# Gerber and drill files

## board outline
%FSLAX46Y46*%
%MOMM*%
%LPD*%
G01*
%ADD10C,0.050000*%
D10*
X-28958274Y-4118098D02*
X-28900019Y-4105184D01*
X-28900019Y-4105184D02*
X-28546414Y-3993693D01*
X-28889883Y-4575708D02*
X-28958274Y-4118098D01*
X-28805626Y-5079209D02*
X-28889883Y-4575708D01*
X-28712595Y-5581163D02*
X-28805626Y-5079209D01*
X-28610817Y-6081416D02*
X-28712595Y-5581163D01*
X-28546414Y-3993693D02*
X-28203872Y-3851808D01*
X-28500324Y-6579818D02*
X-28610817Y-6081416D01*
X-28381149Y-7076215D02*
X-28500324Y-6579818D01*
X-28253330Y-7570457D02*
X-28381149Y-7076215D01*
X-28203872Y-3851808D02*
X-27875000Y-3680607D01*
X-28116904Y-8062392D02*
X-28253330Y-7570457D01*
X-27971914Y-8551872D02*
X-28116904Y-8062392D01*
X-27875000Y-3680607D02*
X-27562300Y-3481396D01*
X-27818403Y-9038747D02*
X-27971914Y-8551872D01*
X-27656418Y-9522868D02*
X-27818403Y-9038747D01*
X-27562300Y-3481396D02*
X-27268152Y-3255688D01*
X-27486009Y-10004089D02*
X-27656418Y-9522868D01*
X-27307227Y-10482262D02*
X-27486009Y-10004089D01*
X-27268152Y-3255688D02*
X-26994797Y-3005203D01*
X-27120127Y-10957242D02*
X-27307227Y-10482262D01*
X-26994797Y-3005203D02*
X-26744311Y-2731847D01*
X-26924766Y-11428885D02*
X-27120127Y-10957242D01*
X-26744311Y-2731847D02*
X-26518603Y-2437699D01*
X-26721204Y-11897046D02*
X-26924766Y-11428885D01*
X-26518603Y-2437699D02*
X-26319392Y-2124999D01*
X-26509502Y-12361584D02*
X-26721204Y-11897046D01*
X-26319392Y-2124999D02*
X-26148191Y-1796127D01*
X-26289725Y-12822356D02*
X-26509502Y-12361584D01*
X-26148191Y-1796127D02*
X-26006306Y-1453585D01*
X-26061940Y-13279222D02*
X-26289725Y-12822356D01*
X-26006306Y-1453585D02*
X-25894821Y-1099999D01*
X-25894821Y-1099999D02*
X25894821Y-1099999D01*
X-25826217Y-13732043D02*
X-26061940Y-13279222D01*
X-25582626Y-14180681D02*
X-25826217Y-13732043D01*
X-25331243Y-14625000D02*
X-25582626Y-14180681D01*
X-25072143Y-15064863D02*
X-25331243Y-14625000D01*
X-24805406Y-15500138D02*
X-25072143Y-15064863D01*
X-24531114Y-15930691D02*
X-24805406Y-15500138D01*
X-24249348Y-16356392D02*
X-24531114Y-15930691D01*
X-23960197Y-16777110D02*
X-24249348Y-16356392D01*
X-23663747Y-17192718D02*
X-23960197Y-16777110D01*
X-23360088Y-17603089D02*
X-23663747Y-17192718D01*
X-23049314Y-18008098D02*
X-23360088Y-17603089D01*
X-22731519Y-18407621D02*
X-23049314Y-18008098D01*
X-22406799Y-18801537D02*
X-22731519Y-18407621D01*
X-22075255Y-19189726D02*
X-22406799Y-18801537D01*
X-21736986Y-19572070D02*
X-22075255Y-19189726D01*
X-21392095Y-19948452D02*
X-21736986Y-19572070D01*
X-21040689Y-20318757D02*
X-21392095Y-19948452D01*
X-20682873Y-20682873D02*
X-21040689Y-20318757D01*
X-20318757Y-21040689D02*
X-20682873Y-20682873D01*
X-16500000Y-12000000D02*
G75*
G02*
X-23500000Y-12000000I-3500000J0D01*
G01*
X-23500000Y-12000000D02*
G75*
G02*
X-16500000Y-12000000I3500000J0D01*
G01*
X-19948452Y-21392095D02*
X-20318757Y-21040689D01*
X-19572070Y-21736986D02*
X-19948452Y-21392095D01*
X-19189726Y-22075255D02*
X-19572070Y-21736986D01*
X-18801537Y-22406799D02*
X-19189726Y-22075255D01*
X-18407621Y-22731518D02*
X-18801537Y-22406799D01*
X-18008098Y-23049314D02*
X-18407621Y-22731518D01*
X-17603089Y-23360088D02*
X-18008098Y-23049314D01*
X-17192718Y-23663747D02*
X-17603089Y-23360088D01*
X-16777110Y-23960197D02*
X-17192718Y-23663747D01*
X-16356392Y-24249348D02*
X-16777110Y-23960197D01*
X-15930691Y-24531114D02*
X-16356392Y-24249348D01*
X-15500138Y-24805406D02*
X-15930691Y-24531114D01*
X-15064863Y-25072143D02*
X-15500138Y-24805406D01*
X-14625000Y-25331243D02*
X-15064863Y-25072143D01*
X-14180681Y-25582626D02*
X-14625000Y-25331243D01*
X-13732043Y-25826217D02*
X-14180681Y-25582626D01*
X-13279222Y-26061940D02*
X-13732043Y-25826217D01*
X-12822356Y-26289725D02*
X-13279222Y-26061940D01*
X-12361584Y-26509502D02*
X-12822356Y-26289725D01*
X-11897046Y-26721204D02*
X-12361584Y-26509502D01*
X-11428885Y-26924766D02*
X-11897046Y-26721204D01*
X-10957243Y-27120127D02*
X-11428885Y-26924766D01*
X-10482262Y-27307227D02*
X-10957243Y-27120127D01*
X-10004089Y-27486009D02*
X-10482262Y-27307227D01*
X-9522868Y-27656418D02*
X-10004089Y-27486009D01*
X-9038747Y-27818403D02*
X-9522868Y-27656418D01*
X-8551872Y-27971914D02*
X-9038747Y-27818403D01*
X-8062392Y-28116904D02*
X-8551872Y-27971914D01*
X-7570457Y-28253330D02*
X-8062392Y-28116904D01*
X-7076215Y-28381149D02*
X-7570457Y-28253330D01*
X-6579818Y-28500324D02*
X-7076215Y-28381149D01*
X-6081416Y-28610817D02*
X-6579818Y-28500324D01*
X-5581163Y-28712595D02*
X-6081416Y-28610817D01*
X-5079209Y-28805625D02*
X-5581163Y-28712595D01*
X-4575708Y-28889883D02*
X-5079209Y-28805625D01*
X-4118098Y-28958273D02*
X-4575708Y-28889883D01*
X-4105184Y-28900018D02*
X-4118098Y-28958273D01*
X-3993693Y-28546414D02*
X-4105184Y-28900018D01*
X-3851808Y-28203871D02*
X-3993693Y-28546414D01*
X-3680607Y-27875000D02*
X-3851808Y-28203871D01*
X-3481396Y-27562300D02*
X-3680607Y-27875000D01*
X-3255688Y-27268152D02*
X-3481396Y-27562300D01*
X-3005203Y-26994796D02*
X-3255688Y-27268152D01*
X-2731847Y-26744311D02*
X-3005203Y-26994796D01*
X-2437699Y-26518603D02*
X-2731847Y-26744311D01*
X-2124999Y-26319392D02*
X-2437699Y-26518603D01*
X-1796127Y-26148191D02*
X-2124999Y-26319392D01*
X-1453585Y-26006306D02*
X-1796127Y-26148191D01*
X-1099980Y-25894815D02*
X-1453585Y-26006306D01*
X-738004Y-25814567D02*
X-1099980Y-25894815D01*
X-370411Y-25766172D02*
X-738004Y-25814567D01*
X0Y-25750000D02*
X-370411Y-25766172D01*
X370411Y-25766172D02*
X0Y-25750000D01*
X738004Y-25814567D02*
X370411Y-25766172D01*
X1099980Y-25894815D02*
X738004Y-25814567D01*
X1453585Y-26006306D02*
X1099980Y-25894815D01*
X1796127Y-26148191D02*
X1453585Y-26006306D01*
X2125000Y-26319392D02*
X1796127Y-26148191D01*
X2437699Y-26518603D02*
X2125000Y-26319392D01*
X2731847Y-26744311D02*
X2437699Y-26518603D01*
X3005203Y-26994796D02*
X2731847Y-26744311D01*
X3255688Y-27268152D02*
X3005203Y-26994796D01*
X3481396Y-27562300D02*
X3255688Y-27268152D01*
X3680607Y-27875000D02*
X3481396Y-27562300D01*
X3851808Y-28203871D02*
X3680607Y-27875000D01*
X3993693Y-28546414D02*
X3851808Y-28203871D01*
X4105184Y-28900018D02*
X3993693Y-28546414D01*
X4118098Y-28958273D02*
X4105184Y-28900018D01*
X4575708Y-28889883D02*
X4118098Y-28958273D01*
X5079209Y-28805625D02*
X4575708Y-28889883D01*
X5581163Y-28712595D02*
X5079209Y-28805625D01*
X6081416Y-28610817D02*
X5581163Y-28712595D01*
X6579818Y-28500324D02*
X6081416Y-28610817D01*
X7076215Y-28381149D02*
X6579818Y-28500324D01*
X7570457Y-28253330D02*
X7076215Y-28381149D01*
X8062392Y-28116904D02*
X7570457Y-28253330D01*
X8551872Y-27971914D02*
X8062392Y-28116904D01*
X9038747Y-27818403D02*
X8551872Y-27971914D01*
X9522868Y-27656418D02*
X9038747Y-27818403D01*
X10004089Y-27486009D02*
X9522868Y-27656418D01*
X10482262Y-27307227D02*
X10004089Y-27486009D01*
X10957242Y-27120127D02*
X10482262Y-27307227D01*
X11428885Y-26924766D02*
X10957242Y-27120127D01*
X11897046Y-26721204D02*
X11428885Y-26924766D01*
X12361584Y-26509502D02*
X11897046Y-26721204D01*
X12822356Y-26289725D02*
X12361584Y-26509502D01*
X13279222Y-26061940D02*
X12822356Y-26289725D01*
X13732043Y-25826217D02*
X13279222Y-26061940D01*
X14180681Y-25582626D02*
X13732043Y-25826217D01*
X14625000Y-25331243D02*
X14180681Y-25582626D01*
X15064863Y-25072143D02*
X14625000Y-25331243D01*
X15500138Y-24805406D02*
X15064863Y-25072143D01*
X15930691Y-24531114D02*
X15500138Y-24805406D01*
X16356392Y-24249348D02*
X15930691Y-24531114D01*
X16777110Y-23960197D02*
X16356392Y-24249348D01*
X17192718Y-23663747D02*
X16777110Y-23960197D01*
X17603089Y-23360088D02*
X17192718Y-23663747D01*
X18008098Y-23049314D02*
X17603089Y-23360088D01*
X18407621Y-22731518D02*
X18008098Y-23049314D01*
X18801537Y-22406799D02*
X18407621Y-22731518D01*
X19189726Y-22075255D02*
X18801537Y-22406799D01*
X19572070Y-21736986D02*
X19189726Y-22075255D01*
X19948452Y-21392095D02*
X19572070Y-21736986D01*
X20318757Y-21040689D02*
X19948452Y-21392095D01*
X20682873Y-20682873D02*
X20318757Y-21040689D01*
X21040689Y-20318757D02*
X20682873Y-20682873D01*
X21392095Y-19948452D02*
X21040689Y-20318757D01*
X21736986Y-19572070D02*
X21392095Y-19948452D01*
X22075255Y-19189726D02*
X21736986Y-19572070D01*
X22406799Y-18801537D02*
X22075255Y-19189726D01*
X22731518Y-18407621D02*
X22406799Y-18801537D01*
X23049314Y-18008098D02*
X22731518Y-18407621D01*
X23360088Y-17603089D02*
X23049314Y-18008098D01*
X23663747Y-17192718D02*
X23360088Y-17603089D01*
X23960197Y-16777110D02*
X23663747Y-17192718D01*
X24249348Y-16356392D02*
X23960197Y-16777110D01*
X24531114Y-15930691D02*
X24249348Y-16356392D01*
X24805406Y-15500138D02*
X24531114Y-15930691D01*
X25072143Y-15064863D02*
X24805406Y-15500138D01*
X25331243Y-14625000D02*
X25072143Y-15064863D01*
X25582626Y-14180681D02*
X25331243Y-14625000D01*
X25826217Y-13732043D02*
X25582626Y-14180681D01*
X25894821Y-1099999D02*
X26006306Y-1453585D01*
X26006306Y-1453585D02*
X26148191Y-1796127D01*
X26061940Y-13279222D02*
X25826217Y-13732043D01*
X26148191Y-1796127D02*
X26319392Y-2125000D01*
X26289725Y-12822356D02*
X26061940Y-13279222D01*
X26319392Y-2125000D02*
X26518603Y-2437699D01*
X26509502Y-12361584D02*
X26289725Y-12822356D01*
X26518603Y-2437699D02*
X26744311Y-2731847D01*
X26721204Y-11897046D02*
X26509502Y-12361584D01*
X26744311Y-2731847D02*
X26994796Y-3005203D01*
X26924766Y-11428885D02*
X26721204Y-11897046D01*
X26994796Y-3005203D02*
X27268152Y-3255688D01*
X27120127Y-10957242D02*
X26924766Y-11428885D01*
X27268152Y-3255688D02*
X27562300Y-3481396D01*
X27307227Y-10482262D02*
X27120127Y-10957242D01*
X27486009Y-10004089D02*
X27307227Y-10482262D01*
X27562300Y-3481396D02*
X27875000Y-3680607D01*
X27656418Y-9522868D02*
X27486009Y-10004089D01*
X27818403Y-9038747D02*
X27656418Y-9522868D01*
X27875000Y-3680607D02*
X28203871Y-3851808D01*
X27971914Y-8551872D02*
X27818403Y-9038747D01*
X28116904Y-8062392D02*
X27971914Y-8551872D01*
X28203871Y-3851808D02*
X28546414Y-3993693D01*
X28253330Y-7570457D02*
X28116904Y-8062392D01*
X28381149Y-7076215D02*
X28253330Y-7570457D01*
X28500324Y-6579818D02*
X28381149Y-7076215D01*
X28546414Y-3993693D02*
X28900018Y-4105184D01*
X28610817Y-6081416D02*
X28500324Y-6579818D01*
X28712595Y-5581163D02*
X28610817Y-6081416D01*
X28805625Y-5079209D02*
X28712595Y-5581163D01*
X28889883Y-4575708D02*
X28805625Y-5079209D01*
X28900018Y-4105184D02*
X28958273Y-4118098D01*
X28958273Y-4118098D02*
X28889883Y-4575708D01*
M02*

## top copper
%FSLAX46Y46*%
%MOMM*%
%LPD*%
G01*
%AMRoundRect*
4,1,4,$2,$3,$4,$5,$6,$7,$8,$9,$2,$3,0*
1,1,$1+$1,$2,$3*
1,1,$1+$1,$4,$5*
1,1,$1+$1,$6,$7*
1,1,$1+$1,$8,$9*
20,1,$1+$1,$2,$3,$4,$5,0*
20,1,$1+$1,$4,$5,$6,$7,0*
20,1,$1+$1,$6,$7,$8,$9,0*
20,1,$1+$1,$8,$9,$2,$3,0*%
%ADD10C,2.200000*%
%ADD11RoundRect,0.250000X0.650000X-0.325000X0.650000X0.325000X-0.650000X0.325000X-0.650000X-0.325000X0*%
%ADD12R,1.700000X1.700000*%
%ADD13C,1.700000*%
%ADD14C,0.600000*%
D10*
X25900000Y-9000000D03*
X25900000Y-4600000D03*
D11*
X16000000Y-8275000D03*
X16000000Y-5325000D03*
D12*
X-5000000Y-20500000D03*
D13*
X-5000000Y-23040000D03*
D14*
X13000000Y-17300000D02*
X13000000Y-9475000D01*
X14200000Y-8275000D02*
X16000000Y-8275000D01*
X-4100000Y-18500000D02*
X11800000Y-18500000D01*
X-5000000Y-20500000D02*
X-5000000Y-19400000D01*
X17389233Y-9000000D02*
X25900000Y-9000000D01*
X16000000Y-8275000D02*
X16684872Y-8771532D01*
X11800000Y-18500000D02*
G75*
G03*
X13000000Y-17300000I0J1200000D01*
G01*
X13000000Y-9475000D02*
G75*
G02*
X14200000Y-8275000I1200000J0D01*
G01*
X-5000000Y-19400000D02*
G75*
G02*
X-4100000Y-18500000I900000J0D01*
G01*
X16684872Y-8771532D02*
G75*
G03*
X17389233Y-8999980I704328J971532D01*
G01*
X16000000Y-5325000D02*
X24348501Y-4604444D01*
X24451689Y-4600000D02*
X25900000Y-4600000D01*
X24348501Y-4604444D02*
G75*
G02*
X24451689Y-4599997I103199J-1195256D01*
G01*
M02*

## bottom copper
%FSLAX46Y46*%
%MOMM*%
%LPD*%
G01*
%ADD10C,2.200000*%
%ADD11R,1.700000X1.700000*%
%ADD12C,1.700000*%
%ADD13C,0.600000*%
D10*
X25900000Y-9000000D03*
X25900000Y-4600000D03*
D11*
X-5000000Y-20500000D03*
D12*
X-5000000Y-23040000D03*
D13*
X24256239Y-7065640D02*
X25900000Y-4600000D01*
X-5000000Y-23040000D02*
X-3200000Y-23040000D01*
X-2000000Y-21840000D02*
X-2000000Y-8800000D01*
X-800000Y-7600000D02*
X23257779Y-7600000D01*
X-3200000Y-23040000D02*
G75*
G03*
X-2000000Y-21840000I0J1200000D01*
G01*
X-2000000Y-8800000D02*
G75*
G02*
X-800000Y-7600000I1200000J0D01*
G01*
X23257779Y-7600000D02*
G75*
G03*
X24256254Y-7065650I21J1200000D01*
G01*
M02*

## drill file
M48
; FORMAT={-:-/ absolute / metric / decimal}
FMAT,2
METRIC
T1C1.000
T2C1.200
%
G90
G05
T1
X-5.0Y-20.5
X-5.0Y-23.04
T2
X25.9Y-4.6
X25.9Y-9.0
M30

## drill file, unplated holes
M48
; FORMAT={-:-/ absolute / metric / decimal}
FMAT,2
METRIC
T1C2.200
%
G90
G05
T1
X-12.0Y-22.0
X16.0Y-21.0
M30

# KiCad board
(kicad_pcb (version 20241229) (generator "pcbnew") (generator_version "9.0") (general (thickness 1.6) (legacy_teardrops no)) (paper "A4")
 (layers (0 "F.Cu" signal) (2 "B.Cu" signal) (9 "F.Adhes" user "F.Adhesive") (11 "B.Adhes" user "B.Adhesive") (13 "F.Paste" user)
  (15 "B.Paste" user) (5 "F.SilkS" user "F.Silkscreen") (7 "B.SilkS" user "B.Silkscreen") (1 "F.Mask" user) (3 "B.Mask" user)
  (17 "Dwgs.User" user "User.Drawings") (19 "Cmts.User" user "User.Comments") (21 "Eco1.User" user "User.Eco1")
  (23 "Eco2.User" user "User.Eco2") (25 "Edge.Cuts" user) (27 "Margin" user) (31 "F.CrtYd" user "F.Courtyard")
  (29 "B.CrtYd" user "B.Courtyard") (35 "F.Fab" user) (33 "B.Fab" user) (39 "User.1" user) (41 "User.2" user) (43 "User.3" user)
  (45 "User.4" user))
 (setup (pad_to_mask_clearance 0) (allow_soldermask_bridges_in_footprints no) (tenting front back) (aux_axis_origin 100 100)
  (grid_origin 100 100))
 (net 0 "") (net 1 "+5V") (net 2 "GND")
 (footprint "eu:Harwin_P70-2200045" (layer "F.Cu") (at 125.9 109)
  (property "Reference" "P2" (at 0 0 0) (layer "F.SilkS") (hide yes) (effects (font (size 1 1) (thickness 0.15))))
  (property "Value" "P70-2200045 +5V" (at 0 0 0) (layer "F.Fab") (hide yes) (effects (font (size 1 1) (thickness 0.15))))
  (pad "1" thru_hole circle (at 0 0) (size 2.2 2.2) (drill 1.2) (layers "*.Cu" "*.Mask" "F.Paste") (remove_unused_layers no) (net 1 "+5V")))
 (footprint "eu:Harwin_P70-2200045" (layer "F.Cu") (at 125.9 104.6)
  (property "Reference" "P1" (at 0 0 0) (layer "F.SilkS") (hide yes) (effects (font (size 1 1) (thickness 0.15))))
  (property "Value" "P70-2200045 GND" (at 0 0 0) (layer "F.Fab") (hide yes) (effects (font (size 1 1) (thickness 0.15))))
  (pad "1" thru_hole circle (at 0 0) (size 2.2 2.2) (drill 1.2) (layers "*.Cu" "*.Mask" "F.Paste") (remove_unused_layers no) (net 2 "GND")))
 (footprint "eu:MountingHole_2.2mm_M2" (layer "F.Cu") (at 88 122)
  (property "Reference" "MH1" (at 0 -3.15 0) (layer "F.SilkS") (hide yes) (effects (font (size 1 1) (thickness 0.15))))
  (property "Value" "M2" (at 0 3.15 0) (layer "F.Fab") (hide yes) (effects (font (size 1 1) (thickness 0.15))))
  (pad "" np_thru_hole circle (at 0 0) (size 2.2 2.2) (drill 2.2) (layers "*.Cu" "*.Mask")))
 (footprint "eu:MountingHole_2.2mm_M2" (layer "F.Cu") (at 116 121)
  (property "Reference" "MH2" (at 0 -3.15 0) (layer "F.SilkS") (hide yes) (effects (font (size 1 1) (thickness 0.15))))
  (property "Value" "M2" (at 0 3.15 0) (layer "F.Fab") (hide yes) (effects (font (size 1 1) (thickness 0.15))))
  (pad "" np_thru_hole circle (at 0 0) (size 2.2 2.2) (drill 2.2) (layers "*.Cu" "*.Mask")))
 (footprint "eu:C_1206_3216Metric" (layer "F.Cu") (at 116 106.8 90)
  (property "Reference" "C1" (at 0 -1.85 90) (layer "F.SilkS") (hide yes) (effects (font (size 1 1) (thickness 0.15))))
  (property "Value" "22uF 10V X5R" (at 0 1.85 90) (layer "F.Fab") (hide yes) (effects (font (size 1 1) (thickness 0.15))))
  (pad "1" smd roundrect (at -1.475 0 90) (size 1.15 1.8) (layers "F.Cu" "F.Mask" "F.Paste") (roundrect_rratio 0.217391) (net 1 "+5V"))
  (pad "2" smd roundrect (at 1.475 0 90) (size 1.15 1.8) (layers "F.Cu" "F.Mask" "F.Paste") (roundrect_rratio 0.217391) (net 2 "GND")))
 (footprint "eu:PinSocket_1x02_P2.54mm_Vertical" (layer "B.Cu") (at 95 120.5 180)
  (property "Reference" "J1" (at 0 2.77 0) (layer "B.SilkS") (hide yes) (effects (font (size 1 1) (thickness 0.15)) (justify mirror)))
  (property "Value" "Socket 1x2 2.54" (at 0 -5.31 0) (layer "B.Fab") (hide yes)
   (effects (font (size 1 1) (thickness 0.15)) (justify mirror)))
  (pad "1" thru_hole rect (at 0 0 180) (size 1.7 1.7) (drill 1) (layers "*.Cu" "*.Mask") (remove_unused_layers no) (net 1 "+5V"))
  (pad "2" thru_hole circle (at 0 -2.54 180) (size 1.7 1.7) (drill 1) (layers "*.Cu" "*.Mask") (remove_unused_layers no) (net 2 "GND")))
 (gr_line (start 71.041726 104.118098) (end 71.099981 104.105184) (stroke (width 0.05) (type default)) (layer "Edge.Cuts"))
 (gr_line (start 71.099981 104.105184) (end 71.453586 103.993693) (stroke (width 0.05) (type default)) (layer "Edge.Cuts"))
 (gr_line (start 71.110117 104.575708) (end 71.041726 104.118098) (stroke (width 0.05) (type default)) (layer "Edge.Cuts"))
 (gr_line (start 71.194374 105.079209) (end 71.110117 104.575708) (stroke (width 0.05) (type default)) (layer "Edge.Cuts"))
 (gr_line (start 71.287405 105.581163) (end 71.194374 105.079209) (stroke (width 0.05) (type default)) (layer "Edge.Cuts"))
 (gr_line (start 71.389183 106.081416) (end 71.287405 105.581163) (stroke (width 0.05) (type default)) (layer "Edge.Cuts"))
 (gr_line (start 71.453586 103.993693) (end 71.796128 103.851808) (stroke (width 0.05) (type default)) (layer "Edge.Cuts"))
 (gr_line (start 71.499676 106.579818) (end 71.389183 106.081416) (stroke (width 0.05) (type default)) (layer "Edge.Cuts"))
 (gr_line (start 71.618851 107.076215) (end 71.499676 106.579818) (stroke (width 0.05) (type default)) (layer "Edge.Cuts"))
 (gr_line (start 71.74667 107.570457) (end 71.618851 107.076215) (stroke (width 0.05) (type default)) (layer "Edge.Cuts"))
 (gr_line (start 71.796128 103.851808) (end 72.125 103.680607) (stroke (width 0.05) (type default)) (layer "Edge.Cuts"))
 (gr_line (start 71.883096 108.062392) (end 71.74667 107.570457) (stroke (width 0.05) (type default)) (layer "Edge.Cuts"))
 (gr_line (start 72.028086 108.551872) (end 71.883096 108.062392) (stroke (width 0.05) (type default)) (layer "Edge.Cuts"))
 (gr_line (start 72.125 103.680607) (end 72.4377 103.481396) (stroke (width 0.05) (type default)) (layer "Edge.Cuts"))
 (gr_line (start 72.181597 109.038747) (end 72.028086 108.551872) (stroke (width 0.05) (type default)) (layer "Edge.Cuts"))
 (gr_line (start 72.343582 109.522868) (end 72.181597 109.038747) (stroke (width 0.05) (type default)) (layer "Edge.Cuts"))
 (gr_line (start 72.4377 103.481396) (end 72.731848 103.255688) (stroke (width 0.05) (type default)) (layer "Edge.Cuts"))
 (gr_line (start 72.513991 110.004089) (end 72.343582 109.522868) (stroke (width 0.05) (type default)) (layer "Edge.Cuts"))
 (gr_line (start 72.692773 110.482262) (end 72.513991 110.004089) (stroke (width 0.05) (type default)) (layer "Edge.Cuts"))
 (gr_line (start 72.731848 103.255688) (end 73.005203 103.005203) (stroke (width 0.05) (type default)) (layer "Edge.Cuts"))
 (gr_line (start 72.879873 110.957242) (end 72.692773 110.482262) (stroke (width 0.05) (type default)) (layer "Edge.Cuts"))
 (gr_line (start 73.005203 103.005203) (end 73.255689 102.731847) (stroke (width 0.05) (type default)) (layer "Edge.Cuts"))
 (gr_line (start 73.075234 111.428885) (end 72.879873 110.957242) (stroke (width 0.05) (type default)) (layer "Edge.Cuts"))
 (gr_line (start 73.255689 102.731847) (end 73.481397 102.437699) (stroke (width 0.05) (type default)) (layer "Edge.Cuts"))
 (gr_line (start 73.278796 111.897046) (end 73.075234 111.428885) (stroke (width 0.05) (type default)) (layer "Edge.Cuts"))
 (gr_line (start 73.481397 102.437699) (end 73.680608 102.124999) (stroke (width 0.05) (type default)) (layer "Edge.Cuts"))
 (gr_line (start 73.490498 112.361584) (end 73.278796 111.897046) (stroke (width 0.05) (type default)) (layer "Edge.Cuts"))
 (gr_line (start 73.680608 102.124999) (end 73.851809 101.796127) (stroke (width 0.05) (type default)) (layer "Edge.Cuts"))
 (gr_line (start 73.710275 112.822356) (end 73.490498 112.361584) (stroke (width 0.05) (type default)) (layer "Edge.Cuts"))
 (gr_line (start 73.851809 101.796127) (end 73.993694 101.453585) (stroke (width 0.05) (type default)) (layer "Edge.Cuts"))
 (gr_line (start 73.93806 113.279222) (end 73.710275 112.822356) (stroke (width 0.05) (type default)) (layer "Edge.Cuts"))
 (gr_line (start 73.993694 101.453585) (end 74.105179 101.099999) (stroke (width 0.05) (type default)) (layer "Edge.Cuts"))
 (gr_line (start 74.105179 101.099999) (end 125.894821 101.099999) (stroke (width 0.05) (type default)) (layer "Edge.Cuts"))
 (gr_line (start 74.173783 113.732043) (end 73.93806 113.279222) (stroke (width 0.05) (type default)) (layer "Edge.Cuts"))
 (gr_line (start 74.417374 114.180681) (end 74.173783 113.732043) (stroke (width 0.05) (type default)) (layer "Edge.Cuts"))
 (gr_line (start 74.668757 114.625) (end 74.417374 114.180681) (stroke (width 0.05) (type default)) (layer "Edge.Cuts"))
 (gr_line (start 74.927857 115.064863) (end 74.668757 114.625) (stroke (width 0.05) (type default)) (layer "Edge.Cuts"))
 (gr_line (start 75.194594 115.500138) (end 74.927857 115.064863) (stroke (width 0.05) (type default)) (layer "Edge.Cuts"))
 (gr_line (start 75.468886 115.930691) (end 75.194594 115.500138) (stroke (width 0.05) (type default)) (layer "Edge.Cuts"))
 (gr_line (start 75.750652 116.356392) (end 75.468886 115.930691) (stroke (width 0.05) (type default)) (layer "Edge.Cuts"))
 (gr_line (start 76.039803 116.77711) (end 75.750652 116.356392) (stroke (width 0.05) (type default)) (layer "Edge.Cuts"))
 (gr_line (start 76.336253 117.192718) (end 76.039803 116.77711) (stroke (width 0.05) (type default)) (layer "Edge.Cuts"))
 (gr_line (start 76.639912 117.603089) (end 76.336253 117.192718) (stroke (width 0.05) (type default)) (layer "Edge.Cuts"))
 (gr_line (start 76.950686 118.008098) (end 76.639912 117.603089) (stroke (width 0.05) (type default)) (layer "Edge.Cuts"))
 (gr_line (start 77.268481 118.407621) (end 76.950686 118.008098) (stroke (width 0.05) (type default)) (layer "Edge.Cuts"))
 (gr_line (start 77.593201 118.801537) (end 77.268481 118.407621) (stroke (width 0.05) (type default)) (layer "Edge.Cuts"))
 (gr_line (start 77.924745 119.189726) (end 77.593201 118.801537) (stroke (width 0.05) (type default)) (layer "Edge.Cuts"))
 (gr_line (start 78.263014 119.57207) (end 77.924745 119.189726) (stroke (width 0.05) (type default)) (layer "Edge.Cuts"))
 (gr_line (start 78.607905 119.948452) (end 78.263014 119.57207) (stroke (width 0.05) (type default)) (layer "Edge.Cuts"))
 (gr_line (start 78.959311 120.318757) (end 78.607905 119.948452) (stroke (width 0.05) (type default)) (layer "Edge.Cuts"))
 (gr_line (start 79.317127 120.682873) (end 78.959311 120.318757) (stroke (width 0.05) (type default)) (layer "Edge.Cuts"))
 (gr_line (start 79.681243 121.040689) (end 79.317127 120.682873) (stroke (width 0.05) (type default)) (layer "Edge.Cuts"))
 (gr_circle (center 80 112) (end 83.5 112) (stroke (width 0.05) (type default)) (fill no) (layer "Edge.Cuts"))
 (gr_line (start 80.051548 121.392095) (end 79.681243 121.040689) (stroke (width 0.05) (type default)) (layer "Edge.Cuts"))
 (gr_line (start 80.42793 121.736986) (end 80.051548 121.392095) (stroke (width 0.05) (type default)) (layer "Edge.Cuts"))
 (gr_line (start 80.810274 122.075255) (end 80.42793 121.736986) (stroke (width 0.05) (type default)) (layer "Edge.Cuts"))
 (gr_line (start 81.198463 122.406799) (end 80.810274 122.075255) (stroke (width 0.05) (type default)) (layer "Edge.Cuts"))
 (gr_line (start 81.592379 122.731518) (end 81.198463 122.406799) (stroke (width 0.05) (type default)) (layer "Edge.Cuts"))
 (gr_line (start 81.991902 123.049314) (end 81.592379 122.731518) (stroke (width 0.05) (type default)) (layer "Edge.Cuts"))
 (gr_line (start 82.396911 123.360088) (end 81.991902 123.049314) (stroke (width 0.05) (type default)) (layer "Edge.Cuts"))
 (gr_line (start 82.807282 123.663747) (end 82.396911 123.360088) (stroke (width 0.05) (type default)) (layer "Edge.Cuts"))
 (gr_line (start 83.22289 123.960197) (end 82.807282 123.663747) (stroke (width 0.05) (type default)) (layer "Edge.Cuts"))
 (gr_line (start 83.643608 124.249348) (end 83.22289 123.960197) (stroke (width 0.05) (type default)) (layer "Edge.Cuts"))
 (gr_line (start 84.069309 124.531114) (end 83.643608 124.249348) (stroke (width 0.05) (type default)) (layer "Edge.Cuts"))
 (gr_line (start 84.499862 124.805406) (end 84.069309 124.531114) (stroke (width 0.05) (type default)) (layer "Edge.Cuts"))
 (gr_line (start 84.935137 125.072143) (end 84.499862 124.805406) (stroke (width 0.05) (type default)) (layer "Edge.Cuts"))
 (gr_line (start 85.375 125.331243) (end 84.935137 125.072143) (stroke (width 0.05) (type default)) (layer "Edge.Cuts"))
 (gr_line (start 85.819319 125.582626) (end 85.375 125.331243) (stroke (width 0.05) (type default)) (layer "Edge.Cuts"))
 (gr_line (start 86.267957 125.826217) (end 85.819319 125.582626) (stroke (width 0.05) (type default)) (layer "Edge.Cuts"))
 (gr_line (start 86.720778 126.06194) (end 86.267957 125.826217) (stroke (width 0.05) (type default)) (layer "Edge.Cuts"))
 (gr_line (start 87.177644 126.289725) (end 86.720778 126.06194) (stroke (width 0.05) (type default)) (layer "Edge.Cuts"))
 (gr_line (start 87.638416 126.509502) (end 87.177644 126.289725) (stroke (width 0.05) (type default)) (layer "Edge.Cuts"))
 (gr_line (start 88.102954 126.721204) (end 87.638416 126.509502) (stroke (width 0.05) (type default)) (layer "Edge.Cuts"))
 (gr_line (start 88.571115 126.924766) (end 88.102954 126.721204) (stroke (width 0.05) (type default)) (layer "Edge.Cuts"))
 (gr_line (start 89.042757 127.120127) (end 88.571115 126.924766) (stroke (width 0.05) (type default)) (layer "Edge.Cuts"))
 (gr_line (start 89.517738 127.307227) (end 89.042757 127.120127) (stroke (width 0.05) (type default)) (layer "Edge.Cuts"))
 (gr_line (start 89.995911 127.486009) (end 89.517738 127.307227) (stroke (width 0.05) (type default)) (layer "Edge.Cuts"))
 (gr_line (start 90.477132 127.656418) (end 89.995911 127.486009) (stroke (width 0.05) (type default)) (layer "Edge.Cuts"))
 (gr_line (start 90.961253 127.818403) (end 90.477132 127.656418) (stroke (width 0.05) (type default)) (layer "Edge.Cuts"))
 (gr_line (start 91.448128 127.971914) (end 90.961253 127.818403) (stroke (width 0.05) (type default)) (layer "Edge.Cuts"))
 (gr_line (start 91.937608 128.116904) (end 91.448128 127.971914) (stroke (width 0.05) (type default)) (layer "Edge.Cuts"))
 (gr_line (start 92.429543 128.25333) (end 91.937608 128.116904) (stroke (width 0.05) (type default)) (layer "Edge.Cuts"))
 (gr_line (start 92.923785 128.381149) (end 92.429543 128.25333) (stroke (width 0.05) (type default)) (layer "Edge.Cuts"))
 (gr_line (start 93.420182 128.500324) (end 92.923785 128.381149) (stroke (width 0.05) (type default)) (layer "Edge.Cuts"))
 (gr_line (start 93.918584 128.610817) (end 93.420182 128.500324) (stroke (width 0.05) (type default)) (layer "Edge.Cuts"))
 (gr_line (start 94.418837 128.712595) (end 93.918584 128.610817) (stroke (width 0.05) (type default)) (layer "Edge.Cuts"))
 (gr_line (start 94.920791 128.805625) (end 94.418837 128.712595) (stroke (width 0.05) (type default)) (layer "Edge.Cuts"))
 (gr_line (start 95.424292 128.889883) (end 94.920791 128.805625) (stroke (width 0.05) (type default)) (layer "Edge.Cuts"))
 (gr_line (start 95.881902 128.958273) (end 95.424292 128.889883) (stroke (width 0.05) (type default)) (layer "Edge.Cuts"))
 (gr_line (start 95.894816 128.900018) (end 95.881902 128.958273) (stroke (width 0.05) (type default)) (layer "Edge.Cuts"))
 (gr_line (start 96.006307 128.546414) (end 95.894816 128.900018) (stroke (width 0.05) (type default)) (layer "Edge.Cuts"))
 (gr_line (start 96.148192 128.203871) (end 96.006307 128.546414) (stroke (width 0.05) (type default)) (layer "Edge.Cuts"))
 (gr_line (start 96.319393 127.875) (end 96.148192 128.203871) (stroke (width 0.05) (type default)) (layer "Edge.Cuts"))
 (gr_line (start 96.518604 127.5623) (end 96.319393 127.875) (stroke (width 0.05) (type default)) (layer "Edge.Cuts"))
 (gr_line (start 96.744312 127.268152) (end 96.518604 127.5623) (stroke (width 0.05) (type default)) (layer "Edge.Cuts"))
 (gr_line (start 96.994797 126.994796) (end 96.744312 127.268152) (stroke (width 0.05) (type default)) (layer "Edge.Cuts"))
 (gr_line (start 97.268153 126.744311) (end 96.994797 126.994796) (stroke (width 0.05) (type default)) (layer "Edge.Cuts"))
 (gr_line (start 97.562301 126.518603) (end 97.268153 126.744311) (stroke (width 0.05) (type default)) (layer "Edge.Cuts"))
 (gr_line (start 97.875001 126.319392) (end 97.562301 126.518603) (stroke (width 0.05) (type default)) (layer "Edge.Cuts"))
 (gr_line (start 98.203873 126.148191) (end 97.875001 126.319392) (stroke (width 0.05) (type default)) (layer "Edge.Cuts"))
 (gr_line (start 98.546415 126.006306) (end 98.203873 126.148191) (stroke (width 0.05) (type default)) (layer "Edge.Cuts"))
 (gr_line (start 98.90002 125.894815) (end 98.546415 126.006306) (stroke (width 0.05) (type default)) (layer "Edge.Cuts"))
 (gr_line (start 99.261996 125.814567) (end 98.90002 125.894815) (stroke (width 0.05) (type default)) (layer "Edge.Cuts"))
 (gr_line (start 99.629589 125.766172) (end 99.261996 125.814567) (stroke (width 0.05) (type default)) (layer "Edge.Cuts"))
 (gr_line (start 100 125.75) (end 99.629589 125.766172) (stroke (width 0.05) (type default)) (layer "Edge.Cuts"))
 (gr_line (start 100.370411 125.766172) (end 100 125.75) (stroke (width 0.05) (type default)) (layer "Edge.Cuts"))
 (gr_line (start 100.738004 125.814567) (end 100.370411 125.766172) (stroke (width 0.05) (type default)) (layer "Edge.Cuts"))
 (gr_line (start 101.09998 125.894815) (end 100.738004 125.814567) (stroke (width 0.05) (type default)) (layer "Edge.Cuts"))
 (gr_line (start 101.453585 126.006306) (end 101.09998 125.894815) (stroke (width 0.05) (type default)) (layer "Edge.Cuts"))
 (gr_line (start 101.796127 126.148191) (end 101.453585 126.006306) (stroke (width 0.05) (type default)) (layer "Edge.Cuts"))
 (gr_line (start 102.125 126.319392) (end 101.796127 126.148191) (stroke (width 0.05) (type default)) (layer "Edge.Cuts"))
 (gr_line (start 102.437699 126.518603) (end 102.125 126.319392) (stroke (width 0.05) (type default)) (layer "Edge.Cuts"))
 (gr_line (start 102.731847 126.744311) (end 102.437699 126.518603) (stroke (width 0.05) (type default)) (layer "Edge.Cuts"))
 (gr_line (start 103.005203 126.994796) (end 102.731847 126.744311) (stroke (width 0.05) (type default)) (layer "Edge.Cuts"))
 (gr_line (start 103.255688 127.268152) (end 103.005203 126.994796) (stroke (width 0.05) (type default)) (layer "Edge.Cuts"))
 (gr_line (start 103.481396 127.5623) (end 103.255688 127.268152) (stroke (width 0.05) (type default)) (layer "Edge.Cuts"))
 (gr_line (start 103.680607 127.875) (end 103.481396 127.5623) (stroke (width 0.05) (type default)) (layer "Edge.Cuts"))
 (gr_line (start 103.851808 128.203871) (end 103.680607 127.875) (stroke (width 0.05) (type default)) (layer "Edge.Cuts"))
 (gr_line (start 103.993693 128.546414) (end 103.851808 128.203871) (stroke (width 0.05) (type default)) (layer "Edge.Cuts"))
 (gr_line (start 104.105184 128.900018) (end 103.993693 128.546414) (stroke (width 0.05) (type default)) (layer "Edge.Cuts"))
 (gr_line (start 104.118098 128.958273) (end 104.105184 128.900018) (stroke (width 0.05) (type default)) (layer "Edge.Cuts"))
 (gr_line (start 104.575708 128.889883) (end 104.118098 128.958273) (stroke (width 0.05) (type default)) (layer "Edge.Cuts"))
 (gr_line (start 105.079209 128.805625) (end 104.575708 128.889883) (stroke (width 0.05) (type default)) (layer "Edge.Cuts"))
 (gr_line (start 105.581163 128.712595) (end 105.079209 128.805625) (stroke (width 0.05) (type default)) (layer "Edge.Cuts"))
 (gr_line (start 106.081416 128.610817) (end 105.581163 128.712595) (stroke (width 0.05) (type default)) (layer "Edge.Cuts"))
 (gr_line (start 106.579818 128.500324) (end 106.081416 128.610817) (stroke (width 0.05) (type default)) (layer "Edge.Cuts"))
 (gr_line (start 107.076215 128.381149) (end 106.579818 128.500324) (stroke (width 0.05) (type default)) (layer "Edge.Cuts"))
 (gr_line (start 107.570457 128.25333) (end 107.076215 128.381149) (stroke (width 0.05) (type default)) (layer "Edge.Cuts"))
 (gr_line (start 108.062392 128.116904) (end 107.570457 128.25333) (stroke (width 0.05) (type default)) (layer "Edge.Cuts"))
 (gr_line (start 108.551872 127.971914) (end 108.062392 128.116904) (stroke (width 0.05) (type default)) (layer "Edge.Cuts"))
 (gr_line (start 109.038747 127.818403) (end 108.551872 127.971914) (stroke (width 0.05) (type default)) (layer "Edge.Cuts"))
 (gr_line (start 109.522868 127.656418) (end 109.038747 127.818403) (stroke (width 0.05) (type default)) (layer "Edge.Cuts"))
 (gr_line (start 110.004089 127.486009) (end 109.522868 127.656418) (stroke (width 0.05) (type default)) (layer "Edge.Cuts"))
 (gr_line (start 110.482262 127.307227) (end 110.004089 127.486009) (stroke (width 0.05) (type default)) (layer "Edge.Cuts"))
 (gr_line (start 110.957242 127.120127) (end 110.482262 127.307227) (stroke (width 0.05) (type default)) (layer "Edge.Cuts"))
 (gr_line (start 111.428885 126.924766) (end 110.957242 127.120127) (stroke (width 0.05) (type default)) (layer "Edge.Cuts"))
 (gr_line (start 111.897046 126.721204) (end 111.428885 126.924766) (stroke (width 0.05) (type default)) (layer "Edge.Cuts"))
 (gr_line (start 112.361584 126.509502) (end 111.897046 126.721204) (stroke (width 0.05) (type default)) (layer "Edge.Cuts"))
 (gr_line (start 112.822356 126.289725) (end 112.361584 126.509502) (stroke (width 0.05) (type default)) (layer "Edge.Cuts"))
 (gr_line (start 113.279222 126.06194) (end 112.822356 126.289725) (stroke (width 0.05) (type default)) (layer "Edge.Cuts"))
 (gr_line (start 113.732043 125.826217) (end 113.279222 126.06194) (stroke (width 0.05) (type default)) (layer "Edge.Cuts"))
 (gr_line (start 114.180681 125.582626) (end 113.732043 125.826217) (stroke (width 0.05) (type default)) (layer "Edge.Cuts"))
 (gr_line (start 114.625 125.331243) (end 114.180681 125.582626) (stroke (width 0.05) (type default)) (layer "Edge.Cuts"))
 (gr_line (start 115.064863 125.072143) (end 114.625 125.331243) (stroke (width 0.05) (type default)) (layer "Edge.Cuts"))
 (gr_line (start 115.500138 124.805406) (end 115.064863 125.072143) (stroke (width 0.05) (type default)) (layer "Edge.Cuts"))
 (gr_line (start 115.930691 124.531114) (end 115.500138 124.805406) (stroke (width 0.05) (type default)) (layer "Edge.Cuts"))
 (gr_line (start 116.356392 124.249348) (end 115.930691 124.531114) (stroke (width 0.05) (type default)) (layer "Edge.Cuts"))
 (gr_line (start 116.77711 123.960197) (end 116.356392 124.249348) (stroke (width 0.05) (type default)) (layer "Edge.Cuts"))
 (gr_line (start 117.192718 123.663747) (end 116.77711 123.960197) (stroke (width 0.05) (type default)) (layer "Edge.Cuts"))
 (gr_line (start 117.603089 123.360088) (end 117.192718 123.663747) (stroke (width 0.05) (type default)) (layer "Edge.Cuts"))
 (gr_line (start 118.008098 123.049314) (end 117.603089 123.360088) (stroke (width 0.05) (type default)) (layer "Edge.Cuts"))
 (gr_line (start 118.407621 122.731518) (end 118.008098 123.049314) (stroke (width 0.05) (type default)) (layer "Edge.Cuts"))
 (gr_line (start 118.801537 122.406799) (end 118.407621 122.731518) (stroke (width 0.05) (type default)) (layer "Edge.Cuts"))
 (gr_line (start 119.189726 122.075255) (end 118.801537 122.406799) (stroke (width 0.05) (type default)) (layer "Edge.Cuts"))
 (gr_line (start 119.57207 121.736986) (end 119.189726 122.075255) (stroke (width 0.05) (type default)) (layer "Edge.Cuts"))
 (gr_line (start 119.948452 121.392095) (end 119.57207 121.736986) (stroke (width 0.05) (type default)) (layer "Edge.Cuts"))
 (gr_line (start 120.318757 121.040689) (end 119.948452 121.392095) (stroke (width 0.05) (type default)) (layer "Edge.Cuts"))
 (gr_line (start 120.682873 120.682873) (end 120.318757 121.040689) (stroke (width 0.05) (type default)) (layer "Edge.Cuts"))
 (gr_line (start 121.040689 120.318757) (end 120.682873 120.682873) (stroke (width 0.05) (type default)) (layer "Edge.Cuts"))
 (gr_line (start 121.392095 119.948452) (end 121.040689 120.318757) (stroke (width 0.05) (type default)) (layer "Edge.Cuts"))
 (gr_line (start 121.736986 119.57207) (end 121.392095 119.948452) (stroke (width 0.05) (type default)) (layer "Edge.Cuts"))
 (gr_line (start 122.075255 119.189726) (end 121.736986 119.57207) (stroke (width 0.05) (type default)) (layer "Edge.Cuts"))
 (gr_line (start 122.406799 118.801537) (end 122.075255 119.189726) (stroke (width 0.05) (type default)) (layer "Edge.Cuts"))
 (gr_line (start 122.731518 118.407621) (end 122.406799 118.801537) (stroke (width 0.05) (type default)) (layer "Edge.Cuts"))
 (gr_line (start 123.049314 118.008098) (end 122.731518 118.407621) (stroke (width 0.05) (type default)) (layer "Edge.Cuts"))
 (gr_line (start 123.360088 117.603089) (end 123.049314 118.008098) (stroke (width 0.05) (type default)) (layer "Edge.Cuts"))
 (gr_line (start 123.663747 117.192718) (end 123.360088 117.603089) (stroke (width 0.05) (type default)) (layer "Edge.Cuts"))
 (gr_line (start 123.960197 116.77711) (end 123.663747 117.192718) (stroke (width 0.05) (type default)) (layer "Edge.Cuts"))
 (gr_line (start 124.249348 116.356392) (end 123.960197 116.77711) (stroke (width 0.05) (type default)) (layer "Edge.Cuts"))
 (gr_line (start 124.531114 115.930691) (end 124.249348 116.356392) (stroke (width 0.05) (type default)) (layer "Edge.Cuts"))
 (gr_line (start 124.805406 115.500138) (end 124.531114 115.930691) (stroke (width 0.05) (type default)) (layer "Edge.Cuts"))
 (gr_line (start 125.072143 115.064863) (end 124.805406 115.500138) (stroke (width 0.05) (type default)) (layer "Edge.Cuts"))
 (gr_line (start 125.331243 114.625) (end 125.072143 115.064863) (stroke (width 0.05) (type default)) (layer "Edge.Cuts"))
 (gr_line (start 125.582626 114.180681) (end 125.331243 114.625) (stroke (width 0.05) (type default)) (layer "Edge.Cuts"))
 (gr_line (start 125.826217 113.732043) (end 125.582626 114.180681) (stroke (width 0.05) (type default)) (layer "Edge.Cuts"))
 (gr_line (start 125.894821 101.099999) (end 126.006306 101.453585) (stroke (width 0.05) (type default)) (layer "Edge.Cuts"))
 (gr_line (start 126.006306 101.453585) (end 126.148191 101.796127) (stroke (width 0.05) (type default)) (layer "Edge.Cuts"))
 (gr_line (start 126.06194 113.279222) (end 125.826217 113.732043) (stroke (width 0.05) (type default)) (layer "Edge.Cuts"))
 (gr_line (start 126.148191 101.796127) (end 126.319392 102.125) (stroke (width 0.05) (type default)) (layer "Edge.Cuts"))
 (gr_line (start 126.289725 112.822356) (end 126.06194 113.279222) (stroke (width 0.05) (type default)) (layer "Edge.Cuts"))
 (gr_line (start 126.319392 102.125) (end 126.518603 102.437699) (stroke (width 0.05) (type default)) (layer "Edge.Cuts"))
 (gr_line (start 126.509502 112.361584) (end 126.289725 112.822356) (stroke (width 0.05) (type default)) (layer "Edge.Cuts"))
 (gr_line (start 126.518603 102.437699) (end 126.744311 102.731847) (stroke (width 0.05) (type default)) (layer "Edge.Cuts"))
 (gr_line (start 126.721204 111.897046) (end 126.509502 112.361584) (stroke (width 0.05) (type default)) (layer "Edge.Cuts"))
 (gr_line (start 126.744311 102.731847) (end 126.994796 103.005203) (stroke (width 0.05) (type default)) (layer "Edge.Cuts"))
 (gr_line (start 126.924766 111.428885) (end 126.721204 111.897046) (stroke (width 0.05) (type default)) (layer "Edge.Cuts"))
 (gr_line (start 126.994796 103.005203) (end 127.268152 103.255688) (stroke (width 0.05) (type default)) (layer "Edge.Cuts"))
 (gr_line (start 127.120127 110.957242) (end 126.924766 111.428885) (stroke (width 0.05) (type default)) (layer "Edge.Cuts"))
 (gr_line (start 127.268152 103.255688) (end 127.5623 103.481396) (stroke (width 0.05) (type default)) (layer "Edge.Cuts"))
 (gr_line (start 127.307227 110.482262) (end 127.120127 110.957242) (stroke (width 0.05) (type default)) (layer "Edge.Cuts"))
 (gr_line (start 127.486009 110.004089) (end 127.307227 110.482262) (stroke (width 0.05) (type default)) (layer "Edge.Cuts"))
 (gr_line (start 127.5623 103.481396) (end 127.875 103.680607) (stroke (width 0.05) (type default)) (layer "Edge.Cuts"))
 (gr_line (start 127.656418 109.522868) (end 127.486009 110.004089) (stroke (width 0.05) (type default)) (layer "Edge.Cuts"))
 (gr_line (start 127.818403 109.038747) (end 127.656418 109.522868) (stroke (width 0.05) (type default)) (layer "Edge.Cuts"))
 (gr_line (start 127.875 103.680607) (end 128.203871 103.851808) (stroke (width 0.05) (type default)) (layer "Edge.Cuts"))
 (gr_line (start 127.971914 108.551872) (end 127.818403 109.038747) (stroke (width 0.05) (type default)) (layer "Edge.Cuts"))
 (gr_line (start 128.116904 108.062392) (end 127.971914 108.551872) (stroke (width 0.05) (type default)) (layer "Edge.Cuts"))
 (gr_line (start 128.203871 103.851808) (end 128.546414 103.993693) (stroke (width 0.05) (type default)) (layer "Edge.Cuts"))
 (gr_line (start 128.25333 107.570457) (end 128.116904 108.062392) (stroke (width 0.05) (type default)) (layer "Edge.Cuts"))
 (gr_line (start 128.381149 107.076215) (end 128.25333 107.570457) (stroke (width 0.05) (type default)) (layer "Edge.Cuts"))
 (gr_line (start 128.500324 106.579818) (end 128.381149 107.076215) (stroke (width 0.05) (type default)) (layer "Edge.Cuts"))
 (gr_line (start 128.546414 103.993693) (end 128.900018 104.105184) (stroke (width 0.05) (type default)) (layer "Edge.Cuts"))
 (gr_line (start 128.610817 106.081416) (end 128.500324 106.579818) (stroke (width 0.05) (type default)) (layer "Edge.Cuts"))
 (gr_line (start 128.712595 105.581163) (end 128.610817 106.081416) (stroke (width 0.05) (type default)) (layer "Edge.Cuts"))
 (gr_line (start 128.805625 105.079209) (end 128.712595 105.581163) (stroke (width 0.05) (type default)) (layer "Edge.Cuts"))
 (gr_line (start 128.889883 104.575708) (end 128.805625 105.079209) (stroke (width 0.05) (type default)) (layer "Edge.Cuts"))
 (gr_line (start 128.900018 104.105184) (end 128.958273 104.118098) (stroke (width 0.05) (type default)) (layer "Edge.Cuts"))
 (gr_line (start 128.958273 104.118098) (end 128.889883 104.575708) (stroke (width 0.05) (type default)) (layer "Edge.Cuts"))
 (segment (start 113 117.3) (end 113 109.475) (width 0.6) (layer "F.Cu") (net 1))
 (segment (start 114.2 108.275) (end 116 108.275) (width 0.6) (layer "F.Cu") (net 1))
 (segment (start 95.9 118.5) (end 111.8 118.5) (width 0.6) (layer "F.Cu") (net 1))
 (segment (start 95 120.5) (end 95 119.4) (width 0.6) (layer "F.Cu") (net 1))
 (segment (start 117.389233 109) (end 125.9 109) (width 0.6) (layer "F.Cu") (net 1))
 (segment (start 116 108.275) (end 116.684872 108.771532) (width 0.6) (layer "F.Cu") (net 1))
 (arc (start 111.8 118.5) (mid 112.648528 118.148528) (end 113 117.3) (width 0.6) (layer "F.Cu") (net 1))
 (arc (start 113 109.475) (mid 113.351471 108.626471) (end 114.2 108.275) (width 0.6) (layer "F.Cu") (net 1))
 (arc (start 95 119.4) (mid 95.263603 118.763603) (end 95.9 118.5) (width 0.6) (layer "F.Cu") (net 1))
 (arc (start 116.684872 108.771532) (mid 117.018989 108.941455) (end 117.389233 109) (width 0.6) (layer "F.Cu") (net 1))
 (segment (start 116 105.325) (end 124.348501 104.604444) (width 0.6) (layer "F.Cu") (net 2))
 (segment (start 124.451689 104.6) (end 125.9 104.6) (width 0.6) (layer "F.Cu") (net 2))
 (arc (start 124.348501 104.604444) (mid 124.400047 104.601111) (end 124.451689 104.6) (width 0.6) (layer "F.Cu") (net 2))
 (segment (start 124.256239 107.06564) (end 125.9 104.6) (width 0.6) (layer "B.Cu") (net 2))
 (segment (start 95 123.04) (end 96.8 123.04) (width 0.6) (layer "B.Cu") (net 2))
 (segment (start 98 121.84) (end 98 108.8) (width 0.6) (layer "B.Cu") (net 2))
 (segment (start 99.2 107.6) (end 123.257779 107.6) (width 0.6) (layer "B.Cu") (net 2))
 (arc (start 96.8 123.04) (mid 97.648528 122.688528) (end 98 121.84) (width 0.6) (layer "B.Cu") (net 2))
 (arc (start 98 108.8) (mid 98.351471 107.951471) (end 99.2 107.6) (width 0.6) (layer "B.Cu") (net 2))
 (arc (start 123.257779 107.6) (mid 123.824009 107.458009) (end 124.256239 107.06564) (width 0.6) (layer "B.Cu") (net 2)))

